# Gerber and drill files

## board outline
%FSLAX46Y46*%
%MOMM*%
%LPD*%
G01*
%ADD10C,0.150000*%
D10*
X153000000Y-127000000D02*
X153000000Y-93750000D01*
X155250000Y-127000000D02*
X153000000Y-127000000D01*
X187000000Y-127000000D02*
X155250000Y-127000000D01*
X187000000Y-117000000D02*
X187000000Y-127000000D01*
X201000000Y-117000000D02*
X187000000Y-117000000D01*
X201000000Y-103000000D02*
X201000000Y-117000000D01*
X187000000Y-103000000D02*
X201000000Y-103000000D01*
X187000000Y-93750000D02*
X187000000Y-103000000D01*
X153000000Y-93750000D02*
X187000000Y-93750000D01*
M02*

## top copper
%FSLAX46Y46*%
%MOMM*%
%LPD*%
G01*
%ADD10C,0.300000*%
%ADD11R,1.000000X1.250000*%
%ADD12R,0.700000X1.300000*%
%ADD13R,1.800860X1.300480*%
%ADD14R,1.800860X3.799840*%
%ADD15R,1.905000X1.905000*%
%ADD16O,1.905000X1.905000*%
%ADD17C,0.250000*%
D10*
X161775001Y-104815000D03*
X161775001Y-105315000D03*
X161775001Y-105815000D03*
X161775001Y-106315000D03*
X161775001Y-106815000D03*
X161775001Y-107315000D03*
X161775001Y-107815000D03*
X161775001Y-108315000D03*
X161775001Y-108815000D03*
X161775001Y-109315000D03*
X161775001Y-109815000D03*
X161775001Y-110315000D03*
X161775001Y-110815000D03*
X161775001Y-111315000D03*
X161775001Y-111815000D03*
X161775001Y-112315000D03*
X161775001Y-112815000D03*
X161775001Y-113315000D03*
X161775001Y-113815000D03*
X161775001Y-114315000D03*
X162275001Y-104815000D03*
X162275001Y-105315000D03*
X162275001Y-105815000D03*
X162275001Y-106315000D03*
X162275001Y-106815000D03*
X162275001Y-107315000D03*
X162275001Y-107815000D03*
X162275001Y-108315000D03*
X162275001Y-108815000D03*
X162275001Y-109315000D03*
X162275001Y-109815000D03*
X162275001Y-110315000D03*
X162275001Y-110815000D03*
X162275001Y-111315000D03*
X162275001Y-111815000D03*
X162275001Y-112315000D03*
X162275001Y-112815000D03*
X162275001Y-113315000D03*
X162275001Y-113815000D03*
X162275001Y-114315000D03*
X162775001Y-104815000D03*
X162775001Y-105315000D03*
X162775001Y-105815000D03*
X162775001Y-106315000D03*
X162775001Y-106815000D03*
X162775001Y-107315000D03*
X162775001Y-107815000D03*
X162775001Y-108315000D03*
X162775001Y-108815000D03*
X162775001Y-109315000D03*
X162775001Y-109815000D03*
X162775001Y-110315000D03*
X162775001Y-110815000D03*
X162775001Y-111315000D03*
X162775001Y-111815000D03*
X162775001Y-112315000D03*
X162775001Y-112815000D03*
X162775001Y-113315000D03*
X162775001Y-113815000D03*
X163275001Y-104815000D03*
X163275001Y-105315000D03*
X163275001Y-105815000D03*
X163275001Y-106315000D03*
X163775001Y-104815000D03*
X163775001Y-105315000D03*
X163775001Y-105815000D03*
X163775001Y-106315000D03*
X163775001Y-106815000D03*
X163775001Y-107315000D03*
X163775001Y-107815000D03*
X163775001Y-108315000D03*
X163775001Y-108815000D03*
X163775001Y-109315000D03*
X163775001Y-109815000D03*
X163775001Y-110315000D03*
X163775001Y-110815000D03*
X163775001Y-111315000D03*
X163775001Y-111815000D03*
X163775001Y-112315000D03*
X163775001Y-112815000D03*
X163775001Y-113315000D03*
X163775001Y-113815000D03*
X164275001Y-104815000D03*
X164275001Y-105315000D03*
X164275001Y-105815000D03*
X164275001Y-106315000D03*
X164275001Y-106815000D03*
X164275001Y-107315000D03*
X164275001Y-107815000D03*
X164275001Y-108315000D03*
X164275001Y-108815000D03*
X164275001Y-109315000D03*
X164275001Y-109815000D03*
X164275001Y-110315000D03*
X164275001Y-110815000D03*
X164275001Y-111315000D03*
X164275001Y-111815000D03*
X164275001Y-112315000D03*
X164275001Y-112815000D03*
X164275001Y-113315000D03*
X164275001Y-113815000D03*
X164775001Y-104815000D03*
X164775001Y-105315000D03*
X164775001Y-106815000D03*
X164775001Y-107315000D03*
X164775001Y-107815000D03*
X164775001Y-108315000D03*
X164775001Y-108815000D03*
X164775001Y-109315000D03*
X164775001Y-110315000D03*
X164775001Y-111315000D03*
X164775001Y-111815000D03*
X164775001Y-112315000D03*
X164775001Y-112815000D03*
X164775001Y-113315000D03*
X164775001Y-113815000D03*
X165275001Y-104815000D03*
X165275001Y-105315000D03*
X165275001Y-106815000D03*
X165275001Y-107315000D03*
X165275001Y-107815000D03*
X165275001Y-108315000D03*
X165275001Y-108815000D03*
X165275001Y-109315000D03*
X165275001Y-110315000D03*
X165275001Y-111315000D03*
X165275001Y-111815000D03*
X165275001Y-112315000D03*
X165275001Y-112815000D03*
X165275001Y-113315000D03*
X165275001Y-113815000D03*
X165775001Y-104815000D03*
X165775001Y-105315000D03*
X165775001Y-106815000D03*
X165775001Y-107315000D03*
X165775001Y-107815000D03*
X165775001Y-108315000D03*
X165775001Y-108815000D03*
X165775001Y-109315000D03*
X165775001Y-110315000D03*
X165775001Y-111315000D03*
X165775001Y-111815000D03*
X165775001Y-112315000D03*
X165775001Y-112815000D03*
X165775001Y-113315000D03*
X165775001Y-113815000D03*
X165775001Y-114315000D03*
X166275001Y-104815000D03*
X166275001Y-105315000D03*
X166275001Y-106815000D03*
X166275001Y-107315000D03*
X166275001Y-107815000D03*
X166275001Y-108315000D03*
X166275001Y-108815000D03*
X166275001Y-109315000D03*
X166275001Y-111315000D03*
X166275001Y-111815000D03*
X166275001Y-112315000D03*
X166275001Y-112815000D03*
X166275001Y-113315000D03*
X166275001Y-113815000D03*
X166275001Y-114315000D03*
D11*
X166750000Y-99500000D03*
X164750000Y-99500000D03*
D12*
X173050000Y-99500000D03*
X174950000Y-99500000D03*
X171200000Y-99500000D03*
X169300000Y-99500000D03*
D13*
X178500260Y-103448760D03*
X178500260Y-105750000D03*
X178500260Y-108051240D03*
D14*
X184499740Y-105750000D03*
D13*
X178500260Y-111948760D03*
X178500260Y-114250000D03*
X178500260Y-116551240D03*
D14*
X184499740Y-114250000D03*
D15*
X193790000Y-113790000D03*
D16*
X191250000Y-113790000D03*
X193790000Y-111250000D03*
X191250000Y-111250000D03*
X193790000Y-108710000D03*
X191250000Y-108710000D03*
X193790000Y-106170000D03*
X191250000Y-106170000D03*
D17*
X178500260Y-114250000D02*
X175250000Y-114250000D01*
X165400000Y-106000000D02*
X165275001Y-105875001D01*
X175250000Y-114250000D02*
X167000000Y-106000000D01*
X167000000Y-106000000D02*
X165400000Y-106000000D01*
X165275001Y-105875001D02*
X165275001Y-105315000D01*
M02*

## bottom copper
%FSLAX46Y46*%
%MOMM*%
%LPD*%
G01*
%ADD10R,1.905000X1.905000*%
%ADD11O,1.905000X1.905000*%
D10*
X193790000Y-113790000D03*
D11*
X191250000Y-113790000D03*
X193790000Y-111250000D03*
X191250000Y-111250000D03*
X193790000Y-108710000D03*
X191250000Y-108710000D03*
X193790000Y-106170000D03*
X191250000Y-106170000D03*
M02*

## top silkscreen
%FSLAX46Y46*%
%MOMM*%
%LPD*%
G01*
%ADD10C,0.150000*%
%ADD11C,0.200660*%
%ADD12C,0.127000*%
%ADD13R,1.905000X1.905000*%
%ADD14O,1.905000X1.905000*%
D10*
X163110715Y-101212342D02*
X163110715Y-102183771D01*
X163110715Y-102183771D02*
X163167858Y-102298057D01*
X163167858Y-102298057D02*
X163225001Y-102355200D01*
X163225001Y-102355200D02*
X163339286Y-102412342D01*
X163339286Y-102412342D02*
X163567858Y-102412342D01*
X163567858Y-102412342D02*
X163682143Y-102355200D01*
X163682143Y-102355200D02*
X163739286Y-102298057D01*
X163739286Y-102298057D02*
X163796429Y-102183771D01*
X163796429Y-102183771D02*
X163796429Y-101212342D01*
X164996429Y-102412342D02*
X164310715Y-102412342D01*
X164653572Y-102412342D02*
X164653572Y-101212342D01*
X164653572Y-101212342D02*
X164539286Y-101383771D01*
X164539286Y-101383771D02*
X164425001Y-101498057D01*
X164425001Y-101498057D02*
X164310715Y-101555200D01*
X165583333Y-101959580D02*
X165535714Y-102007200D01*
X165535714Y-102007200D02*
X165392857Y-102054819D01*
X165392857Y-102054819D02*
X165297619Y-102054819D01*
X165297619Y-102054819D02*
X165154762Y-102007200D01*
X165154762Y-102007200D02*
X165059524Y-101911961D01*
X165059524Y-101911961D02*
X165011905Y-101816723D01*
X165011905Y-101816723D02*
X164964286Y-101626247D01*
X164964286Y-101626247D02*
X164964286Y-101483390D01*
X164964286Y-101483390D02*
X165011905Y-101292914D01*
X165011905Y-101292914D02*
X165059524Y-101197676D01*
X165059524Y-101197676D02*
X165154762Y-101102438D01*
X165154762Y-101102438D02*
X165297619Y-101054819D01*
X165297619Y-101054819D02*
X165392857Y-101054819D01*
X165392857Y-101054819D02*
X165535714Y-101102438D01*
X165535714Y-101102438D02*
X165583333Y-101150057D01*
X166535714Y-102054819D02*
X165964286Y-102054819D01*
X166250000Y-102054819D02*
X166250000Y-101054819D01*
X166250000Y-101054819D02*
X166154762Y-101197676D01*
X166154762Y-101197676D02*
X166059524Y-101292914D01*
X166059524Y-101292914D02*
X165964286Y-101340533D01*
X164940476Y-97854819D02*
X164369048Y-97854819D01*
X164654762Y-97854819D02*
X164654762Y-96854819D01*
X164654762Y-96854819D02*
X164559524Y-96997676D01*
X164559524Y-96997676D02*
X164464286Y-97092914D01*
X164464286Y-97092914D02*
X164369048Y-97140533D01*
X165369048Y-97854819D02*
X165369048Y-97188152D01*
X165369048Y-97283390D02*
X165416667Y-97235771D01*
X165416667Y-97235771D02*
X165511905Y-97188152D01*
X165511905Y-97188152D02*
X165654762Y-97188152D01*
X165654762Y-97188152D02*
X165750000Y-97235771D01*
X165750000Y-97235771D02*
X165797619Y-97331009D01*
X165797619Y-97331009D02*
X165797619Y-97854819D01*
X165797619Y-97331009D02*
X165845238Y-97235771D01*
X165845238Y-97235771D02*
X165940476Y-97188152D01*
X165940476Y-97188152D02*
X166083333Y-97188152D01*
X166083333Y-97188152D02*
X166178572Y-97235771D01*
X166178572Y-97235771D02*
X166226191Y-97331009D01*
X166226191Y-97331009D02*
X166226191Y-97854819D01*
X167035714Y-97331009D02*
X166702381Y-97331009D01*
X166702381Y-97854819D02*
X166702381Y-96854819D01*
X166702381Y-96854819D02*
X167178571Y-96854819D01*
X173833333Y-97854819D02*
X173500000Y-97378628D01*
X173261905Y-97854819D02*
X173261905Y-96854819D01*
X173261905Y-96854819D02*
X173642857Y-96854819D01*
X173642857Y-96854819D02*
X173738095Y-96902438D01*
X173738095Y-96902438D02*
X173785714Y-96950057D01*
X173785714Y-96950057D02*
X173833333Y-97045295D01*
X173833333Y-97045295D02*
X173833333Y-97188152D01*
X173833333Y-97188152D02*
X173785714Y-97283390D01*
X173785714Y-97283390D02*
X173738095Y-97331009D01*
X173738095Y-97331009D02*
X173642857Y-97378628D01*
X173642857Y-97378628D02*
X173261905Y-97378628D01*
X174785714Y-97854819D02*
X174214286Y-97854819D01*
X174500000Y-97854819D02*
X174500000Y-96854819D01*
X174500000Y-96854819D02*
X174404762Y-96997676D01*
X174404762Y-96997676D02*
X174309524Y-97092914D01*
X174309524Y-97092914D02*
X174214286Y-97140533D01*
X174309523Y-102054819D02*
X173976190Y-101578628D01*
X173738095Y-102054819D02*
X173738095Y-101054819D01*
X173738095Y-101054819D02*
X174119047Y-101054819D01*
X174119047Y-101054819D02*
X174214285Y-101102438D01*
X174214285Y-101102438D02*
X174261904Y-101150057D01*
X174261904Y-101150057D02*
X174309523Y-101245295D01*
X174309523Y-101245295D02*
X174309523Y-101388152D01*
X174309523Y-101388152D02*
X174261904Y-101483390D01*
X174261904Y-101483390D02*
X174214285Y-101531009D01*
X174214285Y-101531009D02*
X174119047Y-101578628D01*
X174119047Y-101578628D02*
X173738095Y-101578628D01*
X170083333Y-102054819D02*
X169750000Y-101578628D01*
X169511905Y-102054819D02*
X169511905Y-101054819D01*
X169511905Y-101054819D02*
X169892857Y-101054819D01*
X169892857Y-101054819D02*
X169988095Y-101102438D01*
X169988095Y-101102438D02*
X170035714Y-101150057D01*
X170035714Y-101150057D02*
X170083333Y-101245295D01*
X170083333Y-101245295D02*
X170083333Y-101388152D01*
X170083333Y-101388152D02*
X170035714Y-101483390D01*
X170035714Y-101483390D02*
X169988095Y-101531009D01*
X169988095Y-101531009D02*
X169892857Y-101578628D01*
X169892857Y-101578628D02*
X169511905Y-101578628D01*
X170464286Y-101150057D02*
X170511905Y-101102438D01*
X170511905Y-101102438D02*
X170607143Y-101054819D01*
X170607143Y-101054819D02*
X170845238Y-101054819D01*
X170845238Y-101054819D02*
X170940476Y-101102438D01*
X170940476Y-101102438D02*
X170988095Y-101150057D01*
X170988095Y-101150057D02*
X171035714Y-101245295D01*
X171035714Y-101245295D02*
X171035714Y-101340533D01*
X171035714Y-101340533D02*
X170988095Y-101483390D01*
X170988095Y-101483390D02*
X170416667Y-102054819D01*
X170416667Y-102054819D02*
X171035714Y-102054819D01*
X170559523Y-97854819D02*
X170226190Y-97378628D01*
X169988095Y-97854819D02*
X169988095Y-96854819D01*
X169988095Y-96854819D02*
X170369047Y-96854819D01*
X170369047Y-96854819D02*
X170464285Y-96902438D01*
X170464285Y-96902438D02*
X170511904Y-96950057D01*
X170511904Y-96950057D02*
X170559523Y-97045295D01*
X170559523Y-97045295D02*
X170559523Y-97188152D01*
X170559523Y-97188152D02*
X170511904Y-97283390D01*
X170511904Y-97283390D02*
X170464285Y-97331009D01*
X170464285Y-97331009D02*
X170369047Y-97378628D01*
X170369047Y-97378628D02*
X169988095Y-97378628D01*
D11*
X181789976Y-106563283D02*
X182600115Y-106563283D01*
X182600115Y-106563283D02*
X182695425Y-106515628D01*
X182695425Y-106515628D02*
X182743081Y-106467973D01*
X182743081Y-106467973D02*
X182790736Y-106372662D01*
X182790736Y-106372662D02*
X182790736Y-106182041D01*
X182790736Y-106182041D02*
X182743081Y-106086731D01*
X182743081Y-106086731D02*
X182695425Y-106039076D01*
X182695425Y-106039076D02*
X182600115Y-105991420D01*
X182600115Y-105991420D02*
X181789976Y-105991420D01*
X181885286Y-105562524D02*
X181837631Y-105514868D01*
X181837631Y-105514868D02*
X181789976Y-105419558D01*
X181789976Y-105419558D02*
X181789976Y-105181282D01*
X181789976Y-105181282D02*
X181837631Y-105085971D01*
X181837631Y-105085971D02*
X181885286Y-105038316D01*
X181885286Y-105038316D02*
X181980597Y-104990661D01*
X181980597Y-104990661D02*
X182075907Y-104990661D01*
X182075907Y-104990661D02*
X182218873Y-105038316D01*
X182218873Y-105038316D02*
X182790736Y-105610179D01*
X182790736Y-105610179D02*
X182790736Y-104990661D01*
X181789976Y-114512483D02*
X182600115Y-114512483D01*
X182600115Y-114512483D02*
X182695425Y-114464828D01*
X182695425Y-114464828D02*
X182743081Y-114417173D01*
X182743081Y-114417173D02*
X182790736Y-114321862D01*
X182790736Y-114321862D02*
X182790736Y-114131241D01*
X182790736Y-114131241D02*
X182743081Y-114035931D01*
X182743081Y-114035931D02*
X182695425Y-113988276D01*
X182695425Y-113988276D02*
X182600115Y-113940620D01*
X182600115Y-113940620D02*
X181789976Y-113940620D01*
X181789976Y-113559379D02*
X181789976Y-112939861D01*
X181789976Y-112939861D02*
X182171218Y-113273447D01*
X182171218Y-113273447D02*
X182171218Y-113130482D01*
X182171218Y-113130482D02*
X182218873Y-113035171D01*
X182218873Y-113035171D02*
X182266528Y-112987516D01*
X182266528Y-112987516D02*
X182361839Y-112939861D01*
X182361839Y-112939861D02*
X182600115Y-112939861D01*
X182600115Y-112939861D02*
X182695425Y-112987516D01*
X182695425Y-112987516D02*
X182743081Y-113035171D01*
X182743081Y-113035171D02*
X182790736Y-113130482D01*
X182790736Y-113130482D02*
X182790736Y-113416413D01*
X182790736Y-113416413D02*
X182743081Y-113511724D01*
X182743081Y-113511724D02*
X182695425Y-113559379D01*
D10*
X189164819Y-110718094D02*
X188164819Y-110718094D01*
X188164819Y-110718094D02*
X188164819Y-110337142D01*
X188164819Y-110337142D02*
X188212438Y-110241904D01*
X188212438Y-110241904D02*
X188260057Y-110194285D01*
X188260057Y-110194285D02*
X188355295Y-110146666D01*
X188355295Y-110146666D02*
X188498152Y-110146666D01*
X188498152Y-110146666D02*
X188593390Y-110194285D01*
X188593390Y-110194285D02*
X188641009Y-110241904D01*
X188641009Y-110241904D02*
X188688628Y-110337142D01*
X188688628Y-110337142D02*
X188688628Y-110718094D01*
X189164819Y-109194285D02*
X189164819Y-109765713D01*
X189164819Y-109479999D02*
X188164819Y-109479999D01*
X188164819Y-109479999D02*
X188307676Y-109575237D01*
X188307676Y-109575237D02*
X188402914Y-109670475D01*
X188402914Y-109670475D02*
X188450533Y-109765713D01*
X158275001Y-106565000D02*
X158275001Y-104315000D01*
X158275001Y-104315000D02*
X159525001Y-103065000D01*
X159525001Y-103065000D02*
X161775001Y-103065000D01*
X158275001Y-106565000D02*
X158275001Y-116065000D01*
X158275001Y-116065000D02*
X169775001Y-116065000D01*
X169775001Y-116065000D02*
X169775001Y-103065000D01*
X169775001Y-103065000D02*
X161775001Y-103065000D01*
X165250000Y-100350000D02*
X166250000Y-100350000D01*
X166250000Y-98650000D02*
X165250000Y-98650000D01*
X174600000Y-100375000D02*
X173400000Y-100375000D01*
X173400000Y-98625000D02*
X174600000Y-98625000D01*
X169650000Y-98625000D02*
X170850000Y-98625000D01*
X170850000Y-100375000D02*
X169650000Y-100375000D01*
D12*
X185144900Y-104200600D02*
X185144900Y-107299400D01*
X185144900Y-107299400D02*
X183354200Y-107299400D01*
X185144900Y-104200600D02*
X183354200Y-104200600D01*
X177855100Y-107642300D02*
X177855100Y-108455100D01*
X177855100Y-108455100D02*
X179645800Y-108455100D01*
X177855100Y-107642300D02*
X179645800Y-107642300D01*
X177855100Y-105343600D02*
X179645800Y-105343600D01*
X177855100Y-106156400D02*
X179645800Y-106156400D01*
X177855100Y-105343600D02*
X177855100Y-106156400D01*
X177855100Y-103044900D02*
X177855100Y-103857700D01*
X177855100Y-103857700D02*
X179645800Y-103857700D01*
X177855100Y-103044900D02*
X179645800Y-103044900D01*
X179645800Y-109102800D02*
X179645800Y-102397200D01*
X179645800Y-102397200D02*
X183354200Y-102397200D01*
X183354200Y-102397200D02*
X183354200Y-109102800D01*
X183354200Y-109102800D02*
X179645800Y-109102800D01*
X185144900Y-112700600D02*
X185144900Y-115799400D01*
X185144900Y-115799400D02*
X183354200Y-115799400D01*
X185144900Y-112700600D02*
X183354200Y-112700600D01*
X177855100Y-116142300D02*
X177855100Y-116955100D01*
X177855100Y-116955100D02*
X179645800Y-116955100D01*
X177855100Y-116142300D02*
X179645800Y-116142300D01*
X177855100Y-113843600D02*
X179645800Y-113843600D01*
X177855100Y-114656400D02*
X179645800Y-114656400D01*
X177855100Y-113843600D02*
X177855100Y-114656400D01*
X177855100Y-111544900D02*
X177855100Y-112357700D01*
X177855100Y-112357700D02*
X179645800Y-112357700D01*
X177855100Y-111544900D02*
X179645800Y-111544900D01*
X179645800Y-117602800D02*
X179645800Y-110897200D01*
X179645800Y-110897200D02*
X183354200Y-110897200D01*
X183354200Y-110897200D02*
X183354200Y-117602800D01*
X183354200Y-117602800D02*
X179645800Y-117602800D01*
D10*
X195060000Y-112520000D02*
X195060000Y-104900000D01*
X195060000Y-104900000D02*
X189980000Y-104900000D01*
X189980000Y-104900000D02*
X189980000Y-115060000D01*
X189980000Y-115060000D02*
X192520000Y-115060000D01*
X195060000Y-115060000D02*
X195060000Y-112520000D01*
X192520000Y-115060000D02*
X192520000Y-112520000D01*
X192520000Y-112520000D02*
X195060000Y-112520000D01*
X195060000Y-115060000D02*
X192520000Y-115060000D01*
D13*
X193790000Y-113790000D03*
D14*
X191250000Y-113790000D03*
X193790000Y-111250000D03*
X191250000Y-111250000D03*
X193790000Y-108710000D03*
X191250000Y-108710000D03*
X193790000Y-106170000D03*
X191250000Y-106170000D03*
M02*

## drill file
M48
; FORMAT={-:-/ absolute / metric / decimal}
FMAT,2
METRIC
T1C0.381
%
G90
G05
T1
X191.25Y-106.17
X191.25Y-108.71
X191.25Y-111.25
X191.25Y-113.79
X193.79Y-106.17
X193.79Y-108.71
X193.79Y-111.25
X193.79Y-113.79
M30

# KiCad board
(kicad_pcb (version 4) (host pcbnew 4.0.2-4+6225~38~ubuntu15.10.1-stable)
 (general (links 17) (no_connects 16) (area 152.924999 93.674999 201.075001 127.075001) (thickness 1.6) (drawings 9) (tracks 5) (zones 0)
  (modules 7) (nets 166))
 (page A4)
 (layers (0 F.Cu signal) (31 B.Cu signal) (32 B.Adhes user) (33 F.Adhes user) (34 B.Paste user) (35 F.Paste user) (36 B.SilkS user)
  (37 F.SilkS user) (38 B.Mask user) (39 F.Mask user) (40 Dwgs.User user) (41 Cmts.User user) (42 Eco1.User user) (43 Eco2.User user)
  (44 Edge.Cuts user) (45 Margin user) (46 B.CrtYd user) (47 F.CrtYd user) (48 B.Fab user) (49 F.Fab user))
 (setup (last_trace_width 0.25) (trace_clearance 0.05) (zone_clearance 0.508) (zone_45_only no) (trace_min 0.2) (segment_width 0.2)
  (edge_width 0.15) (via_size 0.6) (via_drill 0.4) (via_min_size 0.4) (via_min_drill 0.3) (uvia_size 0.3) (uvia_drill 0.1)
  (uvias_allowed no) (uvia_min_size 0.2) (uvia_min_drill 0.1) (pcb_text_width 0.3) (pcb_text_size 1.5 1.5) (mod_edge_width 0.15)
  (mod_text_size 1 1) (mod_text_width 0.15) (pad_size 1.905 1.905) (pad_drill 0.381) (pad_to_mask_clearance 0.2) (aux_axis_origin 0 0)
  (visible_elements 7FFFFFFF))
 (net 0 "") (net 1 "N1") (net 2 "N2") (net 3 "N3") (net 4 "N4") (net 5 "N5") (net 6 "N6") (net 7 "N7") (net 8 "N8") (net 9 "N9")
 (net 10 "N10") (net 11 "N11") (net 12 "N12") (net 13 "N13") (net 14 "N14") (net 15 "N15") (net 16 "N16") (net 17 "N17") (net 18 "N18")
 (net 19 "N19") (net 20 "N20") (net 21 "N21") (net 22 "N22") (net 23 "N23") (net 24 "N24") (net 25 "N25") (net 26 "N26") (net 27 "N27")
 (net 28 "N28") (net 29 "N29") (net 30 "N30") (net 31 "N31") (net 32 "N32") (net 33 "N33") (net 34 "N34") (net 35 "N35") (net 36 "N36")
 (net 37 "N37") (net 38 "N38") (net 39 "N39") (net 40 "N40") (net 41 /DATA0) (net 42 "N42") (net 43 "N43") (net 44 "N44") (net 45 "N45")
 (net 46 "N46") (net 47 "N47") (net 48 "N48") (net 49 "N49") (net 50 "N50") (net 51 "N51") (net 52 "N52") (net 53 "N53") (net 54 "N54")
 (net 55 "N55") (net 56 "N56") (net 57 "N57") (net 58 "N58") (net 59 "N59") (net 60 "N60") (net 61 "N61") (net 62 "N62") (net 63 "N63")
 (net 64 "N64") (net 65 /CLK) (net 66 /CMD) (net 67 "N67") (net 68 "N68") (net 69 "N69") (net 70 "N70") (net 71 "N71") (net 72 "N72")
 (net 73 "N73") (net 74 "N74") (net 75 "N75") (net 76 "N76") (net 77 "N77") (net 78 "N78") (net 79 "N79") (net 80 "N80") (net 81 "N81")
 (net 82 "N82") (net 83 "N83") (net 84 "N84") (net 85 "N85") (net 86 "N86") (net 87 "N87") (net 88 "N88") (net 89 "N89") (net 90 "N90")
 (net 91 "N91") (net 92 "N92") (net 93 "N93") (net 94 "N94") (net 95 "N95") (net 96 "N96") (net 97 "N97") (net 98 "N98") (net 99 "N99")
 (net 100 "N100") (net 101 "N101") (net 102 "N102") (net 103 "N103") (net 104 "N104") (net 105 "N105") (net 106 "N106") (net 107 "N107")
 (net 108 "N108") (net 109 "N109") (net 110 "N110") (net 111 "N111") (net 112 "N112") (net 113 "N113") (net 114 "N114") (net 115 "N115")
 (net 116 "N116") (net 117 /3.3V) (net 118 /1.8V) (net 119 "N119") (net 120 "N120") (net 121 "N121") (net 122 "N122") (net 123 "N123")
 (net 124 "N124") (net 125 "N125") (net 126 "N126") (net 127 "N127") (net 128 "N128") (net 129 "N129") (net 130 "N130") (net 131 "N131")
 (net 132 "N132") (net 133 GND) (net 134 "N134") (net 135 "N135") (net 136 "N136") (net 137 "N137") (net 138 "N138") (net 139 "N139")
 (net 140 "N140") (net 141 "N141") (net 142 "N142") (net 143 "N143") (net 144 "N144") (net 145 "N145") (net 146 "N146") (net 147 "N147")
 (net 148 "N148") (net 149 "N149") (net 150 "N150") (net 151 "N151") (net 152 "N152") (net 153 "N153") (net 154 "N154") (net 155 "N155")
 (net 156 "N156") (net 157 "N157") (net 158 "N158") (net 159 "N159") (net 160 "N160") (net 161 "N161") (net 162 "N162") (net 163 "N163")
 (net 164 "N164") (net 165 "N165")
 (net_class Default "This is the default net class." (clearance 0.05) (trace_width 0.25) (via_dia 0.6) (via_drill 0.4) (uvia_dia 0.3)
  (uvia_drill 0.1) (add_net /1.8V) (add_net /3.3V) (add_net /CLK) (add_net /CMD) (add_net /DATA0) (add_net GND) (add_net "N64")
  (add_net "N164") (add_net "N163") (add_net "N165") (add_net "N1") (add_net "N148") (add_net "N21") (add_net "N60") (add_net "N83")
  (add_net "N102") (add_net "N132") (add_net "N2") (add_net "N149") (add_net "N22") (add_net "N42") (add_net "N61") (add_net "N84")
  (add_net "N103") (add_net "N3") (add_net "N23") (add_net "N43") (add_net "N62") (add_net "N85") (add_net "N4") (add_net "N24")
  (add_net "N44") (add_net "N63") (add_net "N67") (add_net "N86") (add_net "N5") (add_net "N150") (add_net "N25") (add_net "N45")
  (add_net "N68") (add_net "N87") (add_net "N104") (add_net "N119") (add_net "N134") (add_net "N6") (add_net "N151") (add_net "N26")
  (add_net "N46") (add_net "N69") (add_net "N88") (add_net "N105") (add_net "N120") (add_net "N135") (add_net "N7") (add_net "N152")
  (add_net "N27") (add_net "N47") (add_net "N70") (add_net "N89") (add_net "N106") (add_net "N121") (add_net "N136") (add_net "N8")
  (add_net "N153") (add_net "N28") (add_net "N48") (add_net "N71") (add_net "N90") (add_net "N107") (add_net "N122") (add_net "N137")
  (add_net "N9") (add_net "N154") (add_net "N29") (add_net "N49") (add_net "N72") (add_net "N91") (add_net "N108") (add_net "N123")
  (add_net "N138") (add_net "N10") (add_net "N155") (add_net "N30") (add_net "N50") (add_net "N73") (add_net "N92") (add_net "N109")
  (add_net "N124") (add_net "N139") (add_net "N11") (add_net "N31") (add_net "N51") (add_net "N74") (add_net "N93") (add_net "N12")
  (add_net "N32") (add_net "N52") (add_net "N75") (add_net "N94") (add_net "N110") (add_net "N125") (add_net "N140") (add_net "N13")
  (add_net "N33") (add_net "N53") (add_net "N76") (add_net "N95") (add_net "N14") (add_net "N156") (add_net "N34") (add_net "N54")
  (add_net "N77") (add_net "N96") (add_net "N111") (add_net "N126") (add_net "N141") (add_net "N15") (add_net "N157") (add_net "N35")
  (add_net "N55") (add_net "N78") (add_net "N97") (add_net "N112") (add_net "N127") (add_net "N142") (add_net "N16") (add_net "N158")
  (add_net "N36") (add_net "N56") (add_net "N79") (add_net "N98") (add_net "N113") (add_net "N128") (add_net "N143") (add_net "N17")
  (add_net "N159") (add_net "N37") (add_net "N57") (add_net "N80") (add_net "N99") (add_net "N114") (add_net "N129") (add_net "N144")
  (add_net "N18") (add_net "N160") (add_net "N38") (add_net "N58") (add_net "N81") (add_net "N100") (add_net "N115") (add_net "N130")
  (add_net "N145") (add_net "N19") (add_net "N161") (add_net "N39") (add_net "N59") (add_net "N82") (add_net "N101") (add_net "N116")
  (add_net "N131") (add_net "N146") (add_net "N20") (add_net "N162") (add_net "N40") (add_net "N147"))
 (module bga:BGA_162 (layer F.Cu) (at 164.025001 109.565)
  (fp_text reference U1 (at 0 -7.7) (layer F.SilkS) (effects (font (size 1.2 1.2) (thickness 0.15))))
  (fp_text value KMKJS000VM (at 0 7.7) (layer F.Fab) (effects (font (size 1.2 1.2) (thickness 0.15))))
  (fp_line (start -5.75 -3) (end -5.75 -5.25) (layer F.SilkS) (width 0.15))
  (fp_line (start -5.75 -5.25) (end -4.5 -6.5) (layer F.SilkS) (width 0.15))
  (fp_line (start -4.5 -6.5) (end -2.25 -6.5) (layer F.SilkS) (width 0.15))
  (fp_line (start -5.75 -3) (end -5.75 6.5) (layer F.SilkS) (width 0.15))
  (fp_line (start -5.75 6.5) (end 5.75 6.5) (layer F.SilkS) (width 0.15))
  (fp_line (start 5.75 6.5) (end 5.75 -6.5) (layer F.SilkS) (width 0.15))
  (fp_line (start 5.75 -6.5) (end -2.25 -6.5) (layer F.SilkS) (width 0.15))
  (pad A1 smd circle (at -2.25 -4.75) (size 0.3 0.3) (layers F.Cu F.Paste F.Mask) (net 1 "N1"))
  (pad B1 smd circle (at -2.25 -4.25) (size 0.3 0.3) (layers F.Cu F.Paste F.Mask) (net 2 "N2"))
  (pad C1 smd circle (at -2.25 -3.75) (size 0.3 0.3) (layers F.Cu F.Paste F.Mask) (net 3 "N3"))
  (pad D1 smd circle (at -2.25 -3.25) (size 0.3 0.3) (layers F.Cu F.Paste F.Mask) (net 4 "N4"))
  (pad E1 smd circle (at -2.25 -2.75) (size 0.3 0.3) (layers F.Cu F.Paste F.Mask) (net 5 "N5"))
  (pad F1 smd circle (at -2.25 -2.25) (size 0.3 0.3) (layers F.Cu F.Paste F.Mask) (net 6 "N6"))
  (pad G1 smd circle (at -2.25 -1.75) (size 0.3 0.3) (layers F.Cu F.Paste F.Mask) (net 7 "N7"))
  (pad H1 smd circle (at -2.25 -1.25) (size 0.3 0.3) (layers F.Cu F.Paste F.Mask) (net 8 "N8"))
  (pad J1 smd circle (at -2.25 -0.75) (size 0.3 0.3) (layers F.Cu F.Paste F.Mask) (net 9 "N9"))
  (pad K1 smd circle (at -2.25 -0.25) (size 0.3 0.3) (layers F.Cu F.Paste F.Mask) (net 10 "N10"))
  (pad L1 smd circle (at -2.25 0.25) (size 0.3 0.3) (layers F.Cu F.Paste F.Mask) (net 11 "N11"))
  (pad M1 smd circle (at -2.25 0.75) (size 0.3 0.3) (layers F.Cu F.Paste F.Mask) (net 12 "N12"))
  (pad N1 smd circle (at -2.25 1.25) (size 0.3 0.3) (layers F.Cu F.Paste F.Mask) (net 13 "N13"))
  (pad P1 smd circle (at -2.25 1.75) (size 0.3 0.3) (layers F.Cu F.Paste F.Mask) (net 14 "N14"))
  (pad R1 smd circle (at -2.25 2.25) (size 0.3 0.3) (layers F.Cu F.Paste F.Mask) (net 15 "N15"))
  (pad T1 smd circle (at -2.25 2.75) (size 0.3 0.3) (layers F.Cu F.Paste F.Mask) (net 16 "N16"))
  (pad U1 smd circle (at -2.25 3.25) (size 0.3 0.3) (layers F.Cu F.Paste F.Mask) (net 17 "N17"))
  (pad V1 smd circle (at -2.25 3.75) (size 0.3 0.3) (layers F.Cu F.Paste F.Mask) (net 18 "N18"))
  (pad W1 smd circle (at -2.25 4.25) (size 0.3 0.3) (layers F.Cu F.Paste F.Mask) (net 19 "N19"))
  (pad Y1 smd circle (at -2.25 4.75) (size 0.3 0.3) (layers F.Cu F.Paste F.Mask) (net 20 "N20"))
  (pad A2 smd circle (at -1.75 -4.75) (size 0.3 0.3) (layers F.Cu F.Paste F.Mask) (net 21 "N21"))
  (pad B2 smd circle (at -1.75 -4.25) (size 0.3 0.3) (layers F.Cu F.Paste F.Mask) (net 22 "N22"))
  (pad C2 smd circle (at -1.75 -3.75) (size 0.3 0.3) (layers F.Cu F.Paste F.Mask) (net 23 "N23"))
  (pad D2 smd circle (at -1.75 -3.25) (size 0.3 0.3) (layers F.Cu F.Paste F.Mask) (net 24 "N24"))
  (pad E2 smd circle (at -1.75 -2.75) (size 0.3 0.3) (layers F.Cu F.Paste F.Mask) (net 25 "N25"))
  (pad F2 smd circle (at -1.75 -2.25) (size 0.3 0.3) (layers F.Cu F.Paste F.Mask) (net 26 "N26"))
  (pad G2 smd circle (at -1.75 -1.75) (size 0.3 0.3) (layers F.Cu F.Paste F.Mask) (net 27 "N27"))
  (pad H2 smd circle (at -1.75 -1.25) (size 0.3 0.3) (layers F.Cu F.Paste F.Mask) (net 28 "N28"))
  (pad J2 smd circle (at -1.75 -0.75) (size 0.3 0.3) (layers F.Cu F.Paste F.Mask) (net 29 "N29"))
  (pad K2 smd circle (at -1.75 -0.25) (size 0.3 0.3) (layers F.Cu F.Paste F.Mask) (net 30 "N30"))
  (pad L2 smd circle (at -1.75 0.25) (size 0.3 0.3) (layers F.Cu F.Paste F.Mask) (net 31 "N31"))
  (pad M2 smd circle (at -1.75 0.75) (size 0.3 0.3) (layers F.Cu F.Paste F.Mask) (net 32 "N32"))
  (pad N2 smd circle (at -1.75 1.25) (size 0.3 0.3) (layers F.Cu F.Paste F.Mask) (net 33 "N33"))
  (pad P2 smd circle (at -1.75 1.75) (size 0.3 0.3) (layers F.Cu F.Paste F.Mask) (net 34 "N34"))
  (pad R2 smd circle (at -1.75 2.25) (size 0.3 0.3) (layers F.Cu F.Paste F.Mask) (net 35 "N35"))
  (pad T2 smd circle (at -1.75 2.75) (size 0.3 0.3) (layers F.Cu F.Paste F.Mask) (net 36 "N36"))
  (pad U2 smd circle (at -1.75 3.25) (size 0.3 0.3) (layers F.Cu F.Paste F.Mask) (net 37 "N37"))
  (pad V2 smd circle (at -1.75 3.75) (size 0.3 0.3) (layers F.Cu F.Paste F.Mask) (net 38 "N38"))
  (pad W2 smd circle (at -1.75 4.25) (size 0.3 0.3) (layers F.Cu F.Paste F.Mask) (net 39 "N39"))
  (pad Y2 smd circle (at -1.75 4.75) (size 0.3 0.3) (layers F.Cu F.Paste F.Mask) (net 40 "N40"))
  (pad A3 smd circle (at -1.25 -4.75) (size 0.3 0.3) (layers F.Cu F.Paste F.Mask) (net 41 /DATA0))
  (pad B3 smd circle (at -1.25 -4.25) (size 0.3 0.3) (layers F.Cu F.Paste F.Mask) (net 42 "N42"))
  (pad C3 smd circle (at -1.25 -3.75) (size 0.3 0.3) (layers F.Cu F.Paste F.Mask) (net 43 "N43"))
  (pad D3 smd circle (at -1.25 -3.25) (size 0.3 0.3) (layers F.Cu F.Paste F.Mask) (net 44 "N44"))
  (pad E3 smd circle (at -1.25 -2.75) (size 0.3 0.3) (layers F.Cu F.Paste F.Mask) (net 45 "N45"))
  (pad F3 smd circle (at -1.25 -2.25) (size 0.3 0.3) (layers F.Cu F.Paste F.Mask) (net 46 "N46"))
  (pad G3 smd circle (at -1.25 -1.75) (size 0.3 0.3) (layers F.Cu F.Paste F.Mask) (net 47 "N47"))
  (pad H3 smd circle (at -1.25 -1.25) (size 0.3 0.3) (layers F.Cu F.Paste F.Mask) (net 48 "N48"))
  (pad J3 smd circle (at -1.25 -0.75) (size 0.3 0.3) (layers F.Cu F.Paste F.Mask) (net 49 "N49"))
  (pad K3 smd circle (at -1.25 -0.25) (size 0.3 0.3) (layers F.Cu F.Paste F.Mask) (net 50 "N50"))
  (pad L3 smd circle (at -1.25 0.25) (size 0.3 0.3) (layers F.Cu F.Paste F.Mask) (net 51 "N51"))
  (pad M3 smd circle (at -1.25 0.75) (size 0.3 0.3) (layers F.Cu F.Paste F.Mask) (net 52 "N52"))
  (pad N3 smd circle (at -1.25 1.25) (size 0.3 0.3) (layers F.Cu F.Paste F.Mask) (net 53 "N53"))
  (pad P3 smd circle (at -1.25 1.75) (size 0.3 0.3) (layers F.Cu F.Paste F.Mask) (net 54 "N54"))
  (pad R3 smd circle (at -1.25 2.25) (size 0.3 0.3) (layers F.Cu F.Paste F.Mask) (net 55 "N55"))
  (pad T3 smd circle (at -1.25 2.75) (size 0.3 0.3) (layers F.Cu F.Paste F.Mask) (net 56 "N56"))
  (pad U3 smd circle (at -1.25 3.25) (size 0.3 0.3) (layers F.Cu F.Paste F.Mask) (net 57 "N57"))
  (pad V3 smd circle (at -1.25 3.75) (size 0.3 0.3) (layers F.Cu F.Paste F.Mask) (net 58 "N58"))
  (pad W3 smd circle (at -1.25 4.25) (size 0.3 0.3) (layers F.Cu F.Paste F.Mask) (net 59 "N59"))
  (pad A4 smd circle (at -0.75 -4.75) (size 0.3 0.3) (layers F.Cu F.Paste F.Mask) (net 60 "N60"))
  (pad B4 smd circle (at -0.75 -4.25) (size 0.3 0.3) (layers F.Cu F.Paste F.Mask) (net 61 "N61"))
  (pad C4 smd circle (at -0.75 -3.75) (size 0.3 0.3) (layers F.Cu F.Paste F.Mask) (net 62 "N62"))
  (pad D4 smd circle (at -0.75 -3.25) (size 0.3 0.3) (layers F.Cu F.Paste F.Mask) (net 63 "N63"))
  (pad A5 smd circle (at -0.25 -4.75) (size 0.3 0.3) (layers F.Cu F.Paste F.Mask) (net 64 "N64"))
  (pad B5 smd circle (at -0.25 -4.25) (size 0.3 0.3) (layers F.Cu F.Paste F.Mask) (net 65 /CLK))
  (pad C5 smd circle (at -0.25 -3.75) (size 0.3 0.3) (layers F.Cu F.Paste F.Mask) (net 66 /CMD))
  (pad D5 smd circle (at -0.25 -3.25) (size 0.3 0.3) (layers F.Cu F.Paste F.Mask) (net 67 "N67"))
  (pad E5 smd circle (at -0.25 -2.75) (size 0.3 0.3) (layers F.Cu F.Paste F.Mask) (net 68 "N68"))
  (pad F5 smd circle (at -0.25 -2.25) (size 0.3 0.3) (layers F.Cu F.Paste F.Mask) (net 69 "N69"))
  (pad G5 smd circle (at -0.25 -1.75) (size 0.3 0.3) (layers F.Cu F.Paste F.Mask) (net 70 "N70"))
  (pad H5 smd circle (at -0.25 -1.25) (size 0.3 0.3) (layers F.Cu F.Paste F.Mask) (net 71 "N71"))
  (pad J5 smd circle (at -0.25 -0.75) (size 0.3 0.3) (layers F.Cu F.Paste F.Mask) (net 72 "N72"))
  (pad K5 smd circle (at -0.25 -0.25) (size 0.3 0.3) (layers F.Cu F.Paste F.Mask) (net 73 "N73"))
  (pad L5 smd circle (at -0.25 0.25) (size 0.3 0.3) (layers F.Cu F.Paste F.Mask) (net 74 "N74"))
  (pad M5 smd circle (at -0.25 0.75) (size 0.3 0.3) (layers F.Cu F.Paste F.Mask) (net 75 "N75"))
  (pad N5 smd circle (at -0.25 1.25) (size 0.3 0.3) (layers F.Cu F.Paste F.Mask) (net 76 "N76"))
  (pad P5 smd circle (at -0.25 1.75) (size 0.3 0.3) (layers F.Cu F.Paste F.Mask) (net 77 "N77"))
  (pad R5 smd circle (at -0.25 2.25) (size 0.3 0.3) (layers F.Cu F.Paste F.Mask) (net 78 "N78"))
  (pad T5 smd circle (at -0.25 2.75) (size 0.3 0.3) (layers F.Cu F.Paste F.Mask) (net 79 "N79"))
  (pad U5 smd circle (at -0.25 3.25) (size 0.3 0.3) (layers F.Cu F.Paste F.Mask) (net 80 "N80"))
  (pad V5 smd circle (at -0.25 3.75) (size 0.3 0.3) (layers F.Cu F.Paste F.Mask) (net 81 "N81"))
  (pad W5 smd circle (at -0.25 4.25) (size 0.3 0.3) (layers F.Cu F.Paste F.Mask) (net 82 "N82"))
  (pad A6 smd circle (at 0.25 -4.75) (size 0.3 0.3) (layers F.Cu F.Paste F.Mask) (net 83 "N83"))
  (pad B6 smd circle (at 0.25 -4.25) (size 0.3 0.3) (layers F.Cu F.Paste F.Mask) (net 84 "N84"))
  (pad C6 smd circle (at 0.25 -3.75) (size 0.3 0.3) (layers F.Cu F.Paste F.Mask) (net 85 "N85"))
  (pad D6 smd circle (at 0.25 -3.25) (size 0.3 0.3) (layers F.Cu F.Paste F.Mask) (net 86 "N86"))
  (pad E6 smd circle (at 0.25 -2.75) (size 0.3 0.3) (layers F.Cu F.Paste F.Mask) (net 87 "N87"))
  (pad F6 smd circle (at 0.25 -2.25) (size 0.3 0.3) (layers F.Cu F.Paste F.Mask) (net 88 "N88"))
  (pad G6 smd circle (at 0.25 -1.75) (size 0.3 0.3) (layers F.Cu F.Paste F.Mask) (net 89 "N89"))
  (pad H6 smd circle (at 0.25 -1.25) (size 0.3 0.3) (layers F.Cu F.Paste F.Mask) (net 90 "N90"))
  (pad J6 smd circle (at 0.25 -0.75) (size 0.3 0.3) (layers F.Cu F.Paste F.Mask) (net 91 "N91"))
  (pad K6 smd circle (at 0.25 -0.25) (size 0.3 0.3) (layers F.Cu F.Paste F.Mask) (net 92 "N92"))
  (pad L6 smd circle (at 0.25 0.25) (size 0.3 0.3) (layers F.Cu F.Paste F.Mask) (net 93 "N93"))
  (pad M6 smd circle (at 0.25 0.75) (size 0.3 0.3) (layers F.Cu F.Paste F.Mask) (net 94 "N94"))
  (pad N6 smd circle (at 0.25 1.25) (size 0.3 0.3) (layers F.Cu F.Paste F.Mask) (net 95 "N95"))
  (pad P6 smd circle (at 0.25 1.75) (size 0.3 0.3) (layers F.Cu F.Paste F.Mask) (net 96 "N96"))
  (pad R6 smd circle (at 0.25 2.25) (size 0.3 0.3) (layers F.Cu F.Paste F.Mask) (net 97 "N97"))
  (pad T6 smd circle (at 0.25 2.75) (size 0.3 0.3) (layers F.Cu F.Paste F.Mask) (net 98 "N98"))
  (pad U6 smd circle (at 0.25 3.25) (size 0.3 0.3) (layers F.Cu F.Paste F.Mask) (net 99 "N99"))
  (pad V6 smd circle (at 0.25 3.75) (size 0.3 0.3) (layers F.Cu F.Paste F.Mask) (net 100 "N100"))
  (pad W6 smd circle (at 0.25 4.25) (size 0.3 0.3) (layers F.Cu F.Paste F.Mask) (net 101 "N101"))
  (pad A7 smd circle (at 0.75 -4.75) (size 0.3 0.3) (layers F.Cu F.Paste F.Mask) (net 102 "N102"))
  (pad B7 smd circle (at 0.75 -4.25) (size 0.3 0.3) (layers F.Cu F.Paste F.Mask) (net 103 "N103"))
  (pad E7 smd circle (at 0.75 -2.75) (size 0.3 0.3) (layers F.Cu F.Paste F.Mask) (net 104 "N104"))
  (pad F7 smd circle (at 0.75 -2.25) (size 0.3 0.3) (layers F.Cu F.Paste F.Mask) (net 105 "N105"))
  (pad G7 smd circle (at 0.75 -1.75) (size 0.3 0.3) (layers F.Cu F.Paste F.Mask) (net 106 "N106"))
  (pad H7 smd circle (at 0.75 -1.25) (size 0.3 0.3) (layers F.Cu F.Paste F.Mask) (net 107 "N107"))
  (pad J7 smd circle (at 0.75 -0.75) (size 0.3 0.3) (layers F.Cu F.Paste F.Mask) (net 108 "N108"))
  (pad K7 smd circle (at 0.75 -0.25) (size 0.3 0.3) (layers F.Cu F.Paste F.Mask) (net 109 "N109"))
  (pad M7 smd circle (at 0.75 0.75) (size 0.3 0.3) (layers F.Cu F.Paste F.Mask) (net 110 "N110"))
  (pad P7 smd circle (at 0.75 1.75) (size 0.3 0.3) (layers F.Cu F.Paste F.Mask) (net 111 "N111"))
  (pad R7 smd circle (at 0.75 2.25) (size 0.3 0.3) (layers F.Cu F.Paste F.Mask) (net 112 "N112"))
  (pad T7 smd circle (at 0.75 2.75) (size 0.3 0.3) (layers F.Cu F.Paste F.Mask) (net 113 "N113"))
  (pad U7 smd circle (at 0.75 3.25) (size 0.3 0.3) (layers F.Cu F.Paste F.Mask) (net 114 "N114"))
  (pad V7 smd circle (at 0.75 3.75) (size 0.3 0.3) (layers F.Cu F.Paste F.Mask) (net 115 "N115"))
  (pad W7 smd circle (at 0.75 4.25) (size 0.3 0.3) (layers F.Cu F.Paste F.Mask) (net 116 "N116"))
  (pad A8 smd circle (at 1.25 -4.75) (size 0.3 0.3) (layers F.Cu F.Paste F.Mask) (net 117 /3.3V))
  (pad B8 smd circle (at 1.25 -4.25) (size 0.3 0.3) (layers F.Cu F.Paste F.Mask) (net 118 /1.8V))
  (pad E8 smd circle (at 1.25 -2.75) (size 0.3 0.3) (layers F.Cu F.Paste F.Mask) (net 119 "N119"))
  (pad F8 smd circle (at 1.25 -2.25) (size 0.3 0.3) (layers F.Cu F.Paste F.Mask) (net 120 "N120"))
  (pad G8 smd circle (at 1.25 -1.75) (size 0.3 0.3) (layers F.Cu F.Paste F.Mask) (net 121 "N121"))
  (pad H8 smd circle (at 1.25 -1.25) (size 0.3 0.3) (layers F.Cu F.Paste F.Mask) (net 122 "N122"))
  (pad J8 smd circle (at 1.25 -0.75) (size 0.3 0.3) (layers F.Cu F.Paste F.Mask) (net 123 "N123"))
  (pad K8 smd circle (at 1.25 -0.25) (size 0.3 0.3) (layers F.Cu F.Paste F.Mask) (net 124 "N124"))
  (pad M8 smd circle (at 1.25 0.75) (size 0.3 0.3) (layers F.Cu F.Paste F.Mask) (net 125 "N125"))
  (pad P8 smd circle (at 1.25 1.75) (size 0.3 0.3) (layers F.Cu F.Paste F.Mask) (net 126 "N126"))
  (pad R8 smd circle (at 1.25 2.25) (size 0.3 0.3) (layers F.Cu F.Paste F.Mask) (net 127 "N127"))
  (pad T8 smd circle (at 1.25 2.75) (size 0.3 0.3) (layers F.Cu F.Paste F.Mask) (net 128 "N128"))
  (pad U8 smd circle (at 1.25 3.25) (size 0.3 0.3) (layers F.Cu F.Paste F.Mask) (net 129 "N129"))
  (pad V8 smd circle (at 1.25 3.75) (size 0.3 0.3) (layers F.Cu F.Paste F.Mask) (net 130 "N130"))
  (pad W8 smd circle (at 1.25 4.25) (size 0.3 0.3) (layers F.Cu F.Paste F.Mask) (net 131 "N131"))
  (pad A9 smd circle (at 1.75 -4.75) (size 0.3 0.3) (layers F.Cu F.Paste F.Mask) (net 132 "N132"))
  (pad B9 smd circle (at 1.75 -4.25) (size 0.3 0.3) (layers F.Cu F.Paste F.Mask) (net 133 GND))
  (pad E9 smd circle (at 1.75 -2.75) (size 0.3 0.3) (layers F.Cu F.Paste F.Mask) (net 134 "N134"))
  (pad F9 smd circle (at 1.75 -2.25) (size 0.3 0.3) (layers F.Cu F.Paste F.Mask) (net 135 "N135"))
  (pad G9 smd circle (at 1.75 -1.75) (size 0.3 0.3) (layers F.Cu F.Paste F.Mask) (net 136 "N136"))
  (pad H9 smd circle (at 1.75 -1.25) (size 0.3 0.3) (layers F.Cu F.Paste F.Mask) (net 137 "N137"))
  (pad J9 smd circle (at 1.75 -0.75) (size 0.3 0.3) (layers F.Cu F.Paste F.Mask) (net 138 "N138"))
  (pad K9 smd circle (at 1.75 -0.25) (size 0.3 0.3) (layers F.Cu F.Paste F.Mask) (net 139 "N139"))
  (pad M9 smd circle (at 1.75 0.75) (size 0.3 0.3) (layers F.Cu F.Paste F.Mask) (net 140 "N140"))
  (pad P9 smd circle (at 1.75 1.75) (size 0.3 0.3) (layers F.Cu F.Paste F.Mask) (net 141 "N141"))
  (pad R9 smd circle (at 1.75 2.25) (size 0.3 0.3) (layers F.Cu F.Paste F.Mask) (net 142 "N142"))
  (pad T9 smd circle (at 1.75 2.75) (size 0.3 0.3) (layers F.Cu F.Paste F.Mask) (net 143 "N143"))
  (pad U9 smd circle (at 1.75 3.25) (size 0.3 0.3) (layers F.Cu F.Paste F.Mask) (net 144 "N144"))
  (pad V9 smd circle (at 1.75 3.75) (size 0.3 0.3) (layers F.Cu F.Paste F.Mask) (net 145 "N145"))
  (pad W9 smd circle (at 1.75 4.25) (size 0.3 0.3) (layers F.Cu F.Paste F.Mask) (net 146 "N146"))
  (pad Y9 smd circle (at 1.75 4.75) (size 0.3 0.3) (layers F.Cu F.Paste F.Mask) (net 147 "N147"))
  (pad A10 smd circle (at 2.25 -4.75) (size 0.3 0.3) (layers F.Cu F.Paste F.Mask) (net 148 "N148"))
  (pad B10 smd circle (at 2.25 -4.25) (size 0.3 0.3) (layers F.Cu F.Paste F.Mask) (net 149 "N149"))
  (pad E10 smd circle (at 2.25 -2.75) (size 0.3 0.3) (layers F.Cu F.Paste F.Mask) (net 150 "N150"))
  (pad F10 smd circle (at 2.25 -2.25) (size 0.3 0.3) (layers F.Cu F.Paste F.Mask) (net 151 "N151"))
  (pad G10 smd circle (at 2.25 -1.75) (size 0.3 0.3) (layers F.Cu F.Paste F.Mask) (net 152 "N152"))
  (pad H10 smd circle (at 2.25 -1.25) (size 0.3 0.3) (layers F.Cu F.Paste F.Mask) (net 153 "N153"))
  (pad J10 smd circle (at 2.25 -0.75) (size 0.3 0.3) (layers F.Cu F.Paste F.Mask) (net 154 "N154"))
  (pad K10 smd circle (at 2.25 -0.25) (size 0.3 0.3) (layers F.Cu F.Paste F.Mask) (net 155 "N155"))
  (pad P10 smd circle (at 2.25 1.75) (size 0.3 0.3) (layers F.Cu F.Paste F.Mask) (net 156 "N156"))
  (pad R10 smd circle (at 2.25 2.25) (size 0.3 0.3) (layers F.Cu F.Paste F.Mask) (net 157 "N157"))
  (pad T10 smd circle (at 2.25 2.75) (size 0.3 0.3) (layers F.Cu F.Paste F.Mask) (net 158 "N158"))
  (pad U10 smd circle (at 2.25 3.25) (size 0.3 0.3) (layers F.Cu F.Paste F.Mask) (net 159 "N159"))
  (pad V10 smd circle (at 2.25 3.75) (size 0.3 0.3) (layers F.Cu F.Paste F.Mask) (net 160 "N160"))
  (pad W10 smd circle (at 2.25 4.25) (size 0.3 0.3) (layers F.Cu F.Paste F.Mask) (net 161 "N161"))
  (pad Y10 smd circle (at 2.25 4.75) (size 0.3 0.3) (layers F.Cu F.Paste F.Mask) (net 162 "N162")))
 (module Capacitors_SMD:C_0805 (layer F.Cu) (at 165.75 99.5 180)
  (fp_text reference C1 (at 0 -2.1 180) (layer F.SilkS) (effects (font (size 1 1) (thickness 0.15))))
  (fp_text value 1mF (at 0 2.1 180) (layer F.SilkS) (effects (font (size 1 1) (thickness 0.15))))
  (fp_line (start 0.5 -0.85) (end -0.5 -0.85) (layer F.SilkS) (width 0.15))
  (fp_line (start -0.5 0.85) (end 0.5 0.85) (layer F.SilkS) (width 0.15))
  (pad 1 smd rect (at -1 0 180) (size 1 1.25) (layers F.Cu F.Paste F.Mask) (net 133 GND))
  (pad 2 smd rect (at 1 0 180) (size 1 1.25) (layers F.Cu F.Paste F.Mask) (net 64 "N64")))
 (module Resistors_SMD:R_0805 (layer F.Cu) (at 174 99.5)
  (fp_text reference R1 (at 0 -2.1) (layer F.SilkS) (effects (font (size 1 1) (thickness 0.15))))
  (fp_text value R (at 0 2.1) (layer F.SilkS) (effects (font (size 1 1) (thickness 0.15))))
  (fp_line (start 0.6 0.875) (end -0.6 0.875) (layer F.SilkS) (width 0.15))
  (fp_line (start -0.6 -0.875) (end 0.6 -0.875) (layer F.SilkS) (width 0.15))
  (pad 1 smd rect (at -0.95 0) (size 0.7 1.3) (layers F.Cu F.Paste F.Mask) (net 118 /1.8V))
  (pad 2 smd rect (at 0.95 0) (size 0.7 1.3) (layers F.Cu F.Paste F.Mask) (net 65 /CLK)))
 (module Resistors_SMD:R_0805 (layer F.Cu) (at 170.25 99.5 180)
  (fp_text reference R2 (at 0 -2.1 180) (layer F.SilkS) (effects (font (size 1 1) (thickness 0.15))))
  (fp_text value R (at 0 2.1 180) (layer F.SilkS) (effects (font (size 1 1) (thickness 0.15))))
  (fp_line (start 0.6 0.875) (end -0.6 0.875) (layer F.SilkS) (width 0.15))
  (fp_line (start -0.6 -0.875) (end 0.6 -0.875) (layer F.SilkS) (width 0.15))
  (pad 1 smd rect (at -0.95 0 180) (size 0.7 1.3) (layers F.Cu F.Paste F.Mask) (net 118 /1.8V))
  (pad 2 smd rect (at 0.95 0 180) (size 0.7 1.3) (layers F.Cu F.Paste F.Mask) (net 41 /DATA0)))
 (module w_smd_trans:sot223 (layer F.Cu) (at 181.5 105.75 270)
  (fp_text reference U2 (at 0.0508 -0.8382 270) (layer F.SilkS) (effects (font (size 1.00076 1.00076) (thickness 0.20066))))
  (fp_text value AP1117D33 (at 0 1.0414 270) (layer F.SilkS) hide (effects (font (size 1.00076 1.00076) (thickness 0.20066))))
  (fp_line (start -1.5494 -3.6449) (end 1.5494 -3.6449) (layer F.SilkS) (width 0.127))
  (fp_line (start 1.5494 -3.6449) (end 1.5494 -1.8542) (layer F.SilkS) (width 0.127))
  (fp_line (start -1.5494 -3.6449) (end -1.5494 -1.8542) (layer F.SilkS) (width 0.127))
  (fp_line (start 1.8923 3.6449) (end 2.7051 3.6449) (layer F.SilkS) (width 0.127))
  (fp_line (start 2.7051 3.6449) (end 2.7051 1.8542) (layer F.SilkS) (width 0.127))
  (fp_line (start 1.8923 3.6449) (end 1.8923 1.8542) (layer F.SilkS) (width 0.127))
  (fp_line (start -0.4064 3.6449) (end -0.4064 1.8542) (layer F.SilkS) (width 0.127))
  (fp_line (start 0.4064 3.6449) (end 0.4064 1.8542) (layer F.SilkS) (width 0.127))
  (fp_line (start -0.4064 3.6449) (end 0.4064 3.6449) (layer F.SilkS) (width 0.127))
  (fp_line (start -2.7051 3.6449) (end -1.8923 3.6449) (layer F.SilkS) (width 0.127))
  (fp_line (start -1.8923 3.6449) (end -1.8923 1.8542) (layer F.SilkS) (width 0.127))
  (fp_line (start -2.7051 3.6449) (end -2.7051 1.8542) (layer F.SilkS) (width 0.127))
  (fp_line (start 3.3528 1.8542) (end -3.3528 1.8542) (layer F.SilkS) (width 0.127))
  (fp_line (start -3.3528 1.8542) (end -3.3528 -1.8542) (layer F.SilkS) (width 0.127))
  (fp_line (start -3.3528 -1.8542) (end 3.3528 -1.8542) (layer F.SilkS) (width 0.127))
  (fp_line (start 3.3528 -1.8542) (end 3.3528 1.8542) (layer F.SilkS) (width 0.127))
  (pad 1 smd rect (at -2.30124 2.99974 270) (size 1.30048 1.80086) (layers F.Cu F.Paste F.Mask) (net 133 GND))
  (pad 2 smd rect (at 0 2.99974 270) (size 1.30048 1.80086) (layers F.Cu F.Paste F.Mask) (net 117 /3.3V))
  (pad 3 smd rect (at 2.30124 2.99974 270) (size 1.30048 1.80086) (layers F.Cu F.Paste F.Mask) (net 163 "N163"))
  (pad 4 smd rect (at 0 -2.99974 270) (size 3.79984 1.80086) (layers F.Cu F.Paste F.Mask)))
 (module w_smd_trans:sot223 (layer F.Cu) (at 181.5 114.25 270)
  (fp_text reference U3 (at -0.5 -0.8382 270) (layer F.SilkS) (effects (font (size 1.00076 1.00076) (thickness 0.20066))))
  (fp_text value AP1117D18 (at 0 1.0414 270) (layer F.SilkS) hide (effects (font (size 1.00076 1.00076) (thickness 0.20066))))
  (fp_line (start -1.5494 -3.6449) (end 1.5494 -3.6449) (layer F.SilkS) (width 0.127))
  (fp_line (start 1.5494 -3.6449) (end 1.5494 -1.8542) (layer F.SilkS) (width 0.127))
  (fp_line (start -1.5494 -3.6449) (end -1.5494 -1.8542) (layer F.SilkS) (width 0.127))
  (fp_line (start 1.8923 3.6449) (end 2.7051 3.6449) (layer F.SilkS) (width 0.127))
  (fp_line (start 2.7051 3.6449) (end 2.7051 1.8542) (layer F.SilkS) (width 0.127))
  (fp_line (start 1.8923 3.6449) (end 1.8923 1.8542) (layer F.SilkS) (width 0.127))
  (fp_line (start -0.4064 3.6449) (end -0.4064 1.8542) (layer F.SilkS) (width 0.127))
  (fp_line (start 0.4064 3.6449) (end 0.4064 1.8542) (layer F.SilkS) (width 0.127))
  (fp_line (start -0.4064 3.6449) (end 0.4064 3.6449) (layer F.SilkS) (width 0.127))
  (fp_line (start -2.7051 3.6449) (end -1.8923 3.6449) (layer F.SilkS) (width 0.127))
  (fp_line (start -1.8923 3.6449) (end -1.8923 1.8542) (layer F.SilkS) (width 0.127))
  (fp_line (start -2.7051 3.6449) (end -2.7051 1.8542) (layer F.SilkS) (width 0.127))
  (fp_line (start 3.3528 1.8542) (end -3.3528 1.8542) (layer F.SilkS) (width 0.127))
  (fp_line (start -3.3528 1.8542) (end -3.3528 -1.8542) (layer F.SilkS) (width 0.127))
  (fp_line (start -3.3528 -1.8542) (end 3.3528 -1.8542) (layer F.SilkS) (width 0.127))
  (fp_line (start 3.3528 -1.8542) (end 3.3528 1.8542) (layer F.SilkS) (width 0.127))
  (pad 1 smd rect (at -2.30124 2.99974 270) (size 1.30048 1.80086) (layers F.Cu F.Paste F.Mask) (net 133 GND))
  (pad 2 smd rect (at 0 2.99974 270) (size 1.30048 1.80086) (layers F.Cu F.Paste F.Mask) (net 118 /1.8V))
  (pad 3 smd rect (at 2.30124 2.99974 270) (size 1.30048 1.80086) (layers F.Cu F.Paste F.Mask) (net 163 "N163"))
  (pad 4 smd rect (at 0 -2.99974 270) (size 3.79984 1.80086) (layers F.Cu F.Paste F.Mask)))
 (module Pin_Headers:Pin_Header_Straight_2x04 (layer F.Cu) (at 192.52 109.98 90)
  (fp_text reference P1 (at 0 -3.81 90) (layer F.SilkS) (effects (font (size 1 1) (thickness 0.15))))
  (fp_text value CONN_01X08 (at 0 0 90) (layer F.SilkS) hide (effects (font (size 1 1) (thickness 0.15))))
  (fp_line (start -2.54 2.54) (end 5.08 2.54) (layer F.SilkS) (width 0.15))
  (fp_line (start 5.08 2.54) (end 5.08 -2.54) (layer F.SilkS) (width 0.15))
  (fp_line (start 5.08 -2.54) (end -5.08 -2.54) (layer F.SilkS) (width 0.15))
  (fp_line (start -5.08 -2.54) (end -5.08 0) (layer F.SilkS) (width 0.15))
  (fp_line (start -5.08 2.54) (end -2.54 2.54) (layer F.SilkS) (width 0.15))
  (fp_line (start -5.08 0) (end -2.54 0) (layer F.SilkS) (width 0.15))
  (fp_line (start -2.54 0) (end -2.54 2.54) (layer F.SilkS) (width 0.15))
  (fp_line (start -5.08 2.54) (end -5.08 0) (layer F.SilkS) (width 0.15))
  (pad 1 thru_hole rect (at -3.81 1.27 90) (size 1.905 1.905) (drill 0.381) (layers *.Cu *.Mask F.SilkS) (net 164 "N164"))
  (pad 2 thru_hole oval (at -3.81 -1.27 90) (size 1.905 1.905) (drill 0.381) (layers *.Cu *.Mask F.SilkS) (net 163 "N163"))
  (pad 3 thru_hole oval (at -1.27 1.27 90) (size 1.905 1.905) (drill 0.381) (layers *.Cu *.Mask F.SilkS) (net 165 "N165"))
  (pad 4 thru_hole oval (at -1.27 -1.27 90) (size 1.905 1.905) (drill 0.381) (layers *.Cu *.Mask F.SilkS) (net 65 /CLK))
  (pad 5 thru_hole oval (at 1.27 1.27 90) (size 1.905 1.905) (drill 0.381) (layers *.Cu *.Mask F.SilkS) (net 66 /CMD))
  (pad 6 thru_hole oval (at 1.27 -1.27 90) (size 1.905 1.905) (drill 0.381) (layers *.Cu *.Mask F.SilkS) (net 65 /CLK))
  (pad 7 thru_hole oval (at 3.81 1.27 90) (size 1.905 1.905) (drill 0.381) (layers *.Cu *.Mask F.SilkS) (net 133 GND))
  (pad 8 thru_hole oval (at 3.81 -1.27 90) (size 1.905 1.905) (drill 0.381) (layers *.Cu *.Mask F.SilkS) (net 41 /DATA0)))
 (gr_line (start 153 127) (end 153 93.75) (angle 90) (layer Edge.Cuts) (width 0.15))
 (gr_line (start 155.25 127) (end 153 127) (angle 90) (layer Edge.Cuts) (width 0.15))
 (gr_line (start 187 127) (end 155.25 127) (angle 90) (layer Edge.Cuts) (width 0.15))
 (gr_line (start 187 117) (end 187 127) (angle 90) (layer Edge.Cuts) (width 0.15))
 (gr_line (start 201 117) (end 187 117) (angle 90) (layer Edge.Cuts) (width 0.15))
 (gr_line (start 201 103) (end 201 117) (angle 90) (layer Edge.Cuts) (width 0.15))
 (gr_line (start 187 103) (end 201 103) (angle 90) (layer Edge.Cuts) (width 0.15))
 (gr_line (start 187 93.75) (end 187 103) (angle 90) (layer Edge.Cuts) (width 0.15))
 (gr_line (start 153 93.75) (end 187 93.75) (angle 90) (layer Edge.Cuts) (width 0.15))
 (segment (start 178.50026 114.25) (end 175.25 114.25) (width 0.25) (layer F.Cu) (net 118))
 (segment (start 165.4 106) (end 165.275001 105.875001) (width 0.25) (layer F.Cu) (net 118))
 (segment (start 175.25 114.25) (end 167 106) (width 0.25) (layer F.Cu) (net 118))
 (segment (start 167 106) (end 165.4 106) (width 0.25) (layer F.Cu) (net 118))
 (segment (start 165.275001 105.875001) (end 165.275001 105.315) (width 0.25) (layer F.Cu) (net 118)))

